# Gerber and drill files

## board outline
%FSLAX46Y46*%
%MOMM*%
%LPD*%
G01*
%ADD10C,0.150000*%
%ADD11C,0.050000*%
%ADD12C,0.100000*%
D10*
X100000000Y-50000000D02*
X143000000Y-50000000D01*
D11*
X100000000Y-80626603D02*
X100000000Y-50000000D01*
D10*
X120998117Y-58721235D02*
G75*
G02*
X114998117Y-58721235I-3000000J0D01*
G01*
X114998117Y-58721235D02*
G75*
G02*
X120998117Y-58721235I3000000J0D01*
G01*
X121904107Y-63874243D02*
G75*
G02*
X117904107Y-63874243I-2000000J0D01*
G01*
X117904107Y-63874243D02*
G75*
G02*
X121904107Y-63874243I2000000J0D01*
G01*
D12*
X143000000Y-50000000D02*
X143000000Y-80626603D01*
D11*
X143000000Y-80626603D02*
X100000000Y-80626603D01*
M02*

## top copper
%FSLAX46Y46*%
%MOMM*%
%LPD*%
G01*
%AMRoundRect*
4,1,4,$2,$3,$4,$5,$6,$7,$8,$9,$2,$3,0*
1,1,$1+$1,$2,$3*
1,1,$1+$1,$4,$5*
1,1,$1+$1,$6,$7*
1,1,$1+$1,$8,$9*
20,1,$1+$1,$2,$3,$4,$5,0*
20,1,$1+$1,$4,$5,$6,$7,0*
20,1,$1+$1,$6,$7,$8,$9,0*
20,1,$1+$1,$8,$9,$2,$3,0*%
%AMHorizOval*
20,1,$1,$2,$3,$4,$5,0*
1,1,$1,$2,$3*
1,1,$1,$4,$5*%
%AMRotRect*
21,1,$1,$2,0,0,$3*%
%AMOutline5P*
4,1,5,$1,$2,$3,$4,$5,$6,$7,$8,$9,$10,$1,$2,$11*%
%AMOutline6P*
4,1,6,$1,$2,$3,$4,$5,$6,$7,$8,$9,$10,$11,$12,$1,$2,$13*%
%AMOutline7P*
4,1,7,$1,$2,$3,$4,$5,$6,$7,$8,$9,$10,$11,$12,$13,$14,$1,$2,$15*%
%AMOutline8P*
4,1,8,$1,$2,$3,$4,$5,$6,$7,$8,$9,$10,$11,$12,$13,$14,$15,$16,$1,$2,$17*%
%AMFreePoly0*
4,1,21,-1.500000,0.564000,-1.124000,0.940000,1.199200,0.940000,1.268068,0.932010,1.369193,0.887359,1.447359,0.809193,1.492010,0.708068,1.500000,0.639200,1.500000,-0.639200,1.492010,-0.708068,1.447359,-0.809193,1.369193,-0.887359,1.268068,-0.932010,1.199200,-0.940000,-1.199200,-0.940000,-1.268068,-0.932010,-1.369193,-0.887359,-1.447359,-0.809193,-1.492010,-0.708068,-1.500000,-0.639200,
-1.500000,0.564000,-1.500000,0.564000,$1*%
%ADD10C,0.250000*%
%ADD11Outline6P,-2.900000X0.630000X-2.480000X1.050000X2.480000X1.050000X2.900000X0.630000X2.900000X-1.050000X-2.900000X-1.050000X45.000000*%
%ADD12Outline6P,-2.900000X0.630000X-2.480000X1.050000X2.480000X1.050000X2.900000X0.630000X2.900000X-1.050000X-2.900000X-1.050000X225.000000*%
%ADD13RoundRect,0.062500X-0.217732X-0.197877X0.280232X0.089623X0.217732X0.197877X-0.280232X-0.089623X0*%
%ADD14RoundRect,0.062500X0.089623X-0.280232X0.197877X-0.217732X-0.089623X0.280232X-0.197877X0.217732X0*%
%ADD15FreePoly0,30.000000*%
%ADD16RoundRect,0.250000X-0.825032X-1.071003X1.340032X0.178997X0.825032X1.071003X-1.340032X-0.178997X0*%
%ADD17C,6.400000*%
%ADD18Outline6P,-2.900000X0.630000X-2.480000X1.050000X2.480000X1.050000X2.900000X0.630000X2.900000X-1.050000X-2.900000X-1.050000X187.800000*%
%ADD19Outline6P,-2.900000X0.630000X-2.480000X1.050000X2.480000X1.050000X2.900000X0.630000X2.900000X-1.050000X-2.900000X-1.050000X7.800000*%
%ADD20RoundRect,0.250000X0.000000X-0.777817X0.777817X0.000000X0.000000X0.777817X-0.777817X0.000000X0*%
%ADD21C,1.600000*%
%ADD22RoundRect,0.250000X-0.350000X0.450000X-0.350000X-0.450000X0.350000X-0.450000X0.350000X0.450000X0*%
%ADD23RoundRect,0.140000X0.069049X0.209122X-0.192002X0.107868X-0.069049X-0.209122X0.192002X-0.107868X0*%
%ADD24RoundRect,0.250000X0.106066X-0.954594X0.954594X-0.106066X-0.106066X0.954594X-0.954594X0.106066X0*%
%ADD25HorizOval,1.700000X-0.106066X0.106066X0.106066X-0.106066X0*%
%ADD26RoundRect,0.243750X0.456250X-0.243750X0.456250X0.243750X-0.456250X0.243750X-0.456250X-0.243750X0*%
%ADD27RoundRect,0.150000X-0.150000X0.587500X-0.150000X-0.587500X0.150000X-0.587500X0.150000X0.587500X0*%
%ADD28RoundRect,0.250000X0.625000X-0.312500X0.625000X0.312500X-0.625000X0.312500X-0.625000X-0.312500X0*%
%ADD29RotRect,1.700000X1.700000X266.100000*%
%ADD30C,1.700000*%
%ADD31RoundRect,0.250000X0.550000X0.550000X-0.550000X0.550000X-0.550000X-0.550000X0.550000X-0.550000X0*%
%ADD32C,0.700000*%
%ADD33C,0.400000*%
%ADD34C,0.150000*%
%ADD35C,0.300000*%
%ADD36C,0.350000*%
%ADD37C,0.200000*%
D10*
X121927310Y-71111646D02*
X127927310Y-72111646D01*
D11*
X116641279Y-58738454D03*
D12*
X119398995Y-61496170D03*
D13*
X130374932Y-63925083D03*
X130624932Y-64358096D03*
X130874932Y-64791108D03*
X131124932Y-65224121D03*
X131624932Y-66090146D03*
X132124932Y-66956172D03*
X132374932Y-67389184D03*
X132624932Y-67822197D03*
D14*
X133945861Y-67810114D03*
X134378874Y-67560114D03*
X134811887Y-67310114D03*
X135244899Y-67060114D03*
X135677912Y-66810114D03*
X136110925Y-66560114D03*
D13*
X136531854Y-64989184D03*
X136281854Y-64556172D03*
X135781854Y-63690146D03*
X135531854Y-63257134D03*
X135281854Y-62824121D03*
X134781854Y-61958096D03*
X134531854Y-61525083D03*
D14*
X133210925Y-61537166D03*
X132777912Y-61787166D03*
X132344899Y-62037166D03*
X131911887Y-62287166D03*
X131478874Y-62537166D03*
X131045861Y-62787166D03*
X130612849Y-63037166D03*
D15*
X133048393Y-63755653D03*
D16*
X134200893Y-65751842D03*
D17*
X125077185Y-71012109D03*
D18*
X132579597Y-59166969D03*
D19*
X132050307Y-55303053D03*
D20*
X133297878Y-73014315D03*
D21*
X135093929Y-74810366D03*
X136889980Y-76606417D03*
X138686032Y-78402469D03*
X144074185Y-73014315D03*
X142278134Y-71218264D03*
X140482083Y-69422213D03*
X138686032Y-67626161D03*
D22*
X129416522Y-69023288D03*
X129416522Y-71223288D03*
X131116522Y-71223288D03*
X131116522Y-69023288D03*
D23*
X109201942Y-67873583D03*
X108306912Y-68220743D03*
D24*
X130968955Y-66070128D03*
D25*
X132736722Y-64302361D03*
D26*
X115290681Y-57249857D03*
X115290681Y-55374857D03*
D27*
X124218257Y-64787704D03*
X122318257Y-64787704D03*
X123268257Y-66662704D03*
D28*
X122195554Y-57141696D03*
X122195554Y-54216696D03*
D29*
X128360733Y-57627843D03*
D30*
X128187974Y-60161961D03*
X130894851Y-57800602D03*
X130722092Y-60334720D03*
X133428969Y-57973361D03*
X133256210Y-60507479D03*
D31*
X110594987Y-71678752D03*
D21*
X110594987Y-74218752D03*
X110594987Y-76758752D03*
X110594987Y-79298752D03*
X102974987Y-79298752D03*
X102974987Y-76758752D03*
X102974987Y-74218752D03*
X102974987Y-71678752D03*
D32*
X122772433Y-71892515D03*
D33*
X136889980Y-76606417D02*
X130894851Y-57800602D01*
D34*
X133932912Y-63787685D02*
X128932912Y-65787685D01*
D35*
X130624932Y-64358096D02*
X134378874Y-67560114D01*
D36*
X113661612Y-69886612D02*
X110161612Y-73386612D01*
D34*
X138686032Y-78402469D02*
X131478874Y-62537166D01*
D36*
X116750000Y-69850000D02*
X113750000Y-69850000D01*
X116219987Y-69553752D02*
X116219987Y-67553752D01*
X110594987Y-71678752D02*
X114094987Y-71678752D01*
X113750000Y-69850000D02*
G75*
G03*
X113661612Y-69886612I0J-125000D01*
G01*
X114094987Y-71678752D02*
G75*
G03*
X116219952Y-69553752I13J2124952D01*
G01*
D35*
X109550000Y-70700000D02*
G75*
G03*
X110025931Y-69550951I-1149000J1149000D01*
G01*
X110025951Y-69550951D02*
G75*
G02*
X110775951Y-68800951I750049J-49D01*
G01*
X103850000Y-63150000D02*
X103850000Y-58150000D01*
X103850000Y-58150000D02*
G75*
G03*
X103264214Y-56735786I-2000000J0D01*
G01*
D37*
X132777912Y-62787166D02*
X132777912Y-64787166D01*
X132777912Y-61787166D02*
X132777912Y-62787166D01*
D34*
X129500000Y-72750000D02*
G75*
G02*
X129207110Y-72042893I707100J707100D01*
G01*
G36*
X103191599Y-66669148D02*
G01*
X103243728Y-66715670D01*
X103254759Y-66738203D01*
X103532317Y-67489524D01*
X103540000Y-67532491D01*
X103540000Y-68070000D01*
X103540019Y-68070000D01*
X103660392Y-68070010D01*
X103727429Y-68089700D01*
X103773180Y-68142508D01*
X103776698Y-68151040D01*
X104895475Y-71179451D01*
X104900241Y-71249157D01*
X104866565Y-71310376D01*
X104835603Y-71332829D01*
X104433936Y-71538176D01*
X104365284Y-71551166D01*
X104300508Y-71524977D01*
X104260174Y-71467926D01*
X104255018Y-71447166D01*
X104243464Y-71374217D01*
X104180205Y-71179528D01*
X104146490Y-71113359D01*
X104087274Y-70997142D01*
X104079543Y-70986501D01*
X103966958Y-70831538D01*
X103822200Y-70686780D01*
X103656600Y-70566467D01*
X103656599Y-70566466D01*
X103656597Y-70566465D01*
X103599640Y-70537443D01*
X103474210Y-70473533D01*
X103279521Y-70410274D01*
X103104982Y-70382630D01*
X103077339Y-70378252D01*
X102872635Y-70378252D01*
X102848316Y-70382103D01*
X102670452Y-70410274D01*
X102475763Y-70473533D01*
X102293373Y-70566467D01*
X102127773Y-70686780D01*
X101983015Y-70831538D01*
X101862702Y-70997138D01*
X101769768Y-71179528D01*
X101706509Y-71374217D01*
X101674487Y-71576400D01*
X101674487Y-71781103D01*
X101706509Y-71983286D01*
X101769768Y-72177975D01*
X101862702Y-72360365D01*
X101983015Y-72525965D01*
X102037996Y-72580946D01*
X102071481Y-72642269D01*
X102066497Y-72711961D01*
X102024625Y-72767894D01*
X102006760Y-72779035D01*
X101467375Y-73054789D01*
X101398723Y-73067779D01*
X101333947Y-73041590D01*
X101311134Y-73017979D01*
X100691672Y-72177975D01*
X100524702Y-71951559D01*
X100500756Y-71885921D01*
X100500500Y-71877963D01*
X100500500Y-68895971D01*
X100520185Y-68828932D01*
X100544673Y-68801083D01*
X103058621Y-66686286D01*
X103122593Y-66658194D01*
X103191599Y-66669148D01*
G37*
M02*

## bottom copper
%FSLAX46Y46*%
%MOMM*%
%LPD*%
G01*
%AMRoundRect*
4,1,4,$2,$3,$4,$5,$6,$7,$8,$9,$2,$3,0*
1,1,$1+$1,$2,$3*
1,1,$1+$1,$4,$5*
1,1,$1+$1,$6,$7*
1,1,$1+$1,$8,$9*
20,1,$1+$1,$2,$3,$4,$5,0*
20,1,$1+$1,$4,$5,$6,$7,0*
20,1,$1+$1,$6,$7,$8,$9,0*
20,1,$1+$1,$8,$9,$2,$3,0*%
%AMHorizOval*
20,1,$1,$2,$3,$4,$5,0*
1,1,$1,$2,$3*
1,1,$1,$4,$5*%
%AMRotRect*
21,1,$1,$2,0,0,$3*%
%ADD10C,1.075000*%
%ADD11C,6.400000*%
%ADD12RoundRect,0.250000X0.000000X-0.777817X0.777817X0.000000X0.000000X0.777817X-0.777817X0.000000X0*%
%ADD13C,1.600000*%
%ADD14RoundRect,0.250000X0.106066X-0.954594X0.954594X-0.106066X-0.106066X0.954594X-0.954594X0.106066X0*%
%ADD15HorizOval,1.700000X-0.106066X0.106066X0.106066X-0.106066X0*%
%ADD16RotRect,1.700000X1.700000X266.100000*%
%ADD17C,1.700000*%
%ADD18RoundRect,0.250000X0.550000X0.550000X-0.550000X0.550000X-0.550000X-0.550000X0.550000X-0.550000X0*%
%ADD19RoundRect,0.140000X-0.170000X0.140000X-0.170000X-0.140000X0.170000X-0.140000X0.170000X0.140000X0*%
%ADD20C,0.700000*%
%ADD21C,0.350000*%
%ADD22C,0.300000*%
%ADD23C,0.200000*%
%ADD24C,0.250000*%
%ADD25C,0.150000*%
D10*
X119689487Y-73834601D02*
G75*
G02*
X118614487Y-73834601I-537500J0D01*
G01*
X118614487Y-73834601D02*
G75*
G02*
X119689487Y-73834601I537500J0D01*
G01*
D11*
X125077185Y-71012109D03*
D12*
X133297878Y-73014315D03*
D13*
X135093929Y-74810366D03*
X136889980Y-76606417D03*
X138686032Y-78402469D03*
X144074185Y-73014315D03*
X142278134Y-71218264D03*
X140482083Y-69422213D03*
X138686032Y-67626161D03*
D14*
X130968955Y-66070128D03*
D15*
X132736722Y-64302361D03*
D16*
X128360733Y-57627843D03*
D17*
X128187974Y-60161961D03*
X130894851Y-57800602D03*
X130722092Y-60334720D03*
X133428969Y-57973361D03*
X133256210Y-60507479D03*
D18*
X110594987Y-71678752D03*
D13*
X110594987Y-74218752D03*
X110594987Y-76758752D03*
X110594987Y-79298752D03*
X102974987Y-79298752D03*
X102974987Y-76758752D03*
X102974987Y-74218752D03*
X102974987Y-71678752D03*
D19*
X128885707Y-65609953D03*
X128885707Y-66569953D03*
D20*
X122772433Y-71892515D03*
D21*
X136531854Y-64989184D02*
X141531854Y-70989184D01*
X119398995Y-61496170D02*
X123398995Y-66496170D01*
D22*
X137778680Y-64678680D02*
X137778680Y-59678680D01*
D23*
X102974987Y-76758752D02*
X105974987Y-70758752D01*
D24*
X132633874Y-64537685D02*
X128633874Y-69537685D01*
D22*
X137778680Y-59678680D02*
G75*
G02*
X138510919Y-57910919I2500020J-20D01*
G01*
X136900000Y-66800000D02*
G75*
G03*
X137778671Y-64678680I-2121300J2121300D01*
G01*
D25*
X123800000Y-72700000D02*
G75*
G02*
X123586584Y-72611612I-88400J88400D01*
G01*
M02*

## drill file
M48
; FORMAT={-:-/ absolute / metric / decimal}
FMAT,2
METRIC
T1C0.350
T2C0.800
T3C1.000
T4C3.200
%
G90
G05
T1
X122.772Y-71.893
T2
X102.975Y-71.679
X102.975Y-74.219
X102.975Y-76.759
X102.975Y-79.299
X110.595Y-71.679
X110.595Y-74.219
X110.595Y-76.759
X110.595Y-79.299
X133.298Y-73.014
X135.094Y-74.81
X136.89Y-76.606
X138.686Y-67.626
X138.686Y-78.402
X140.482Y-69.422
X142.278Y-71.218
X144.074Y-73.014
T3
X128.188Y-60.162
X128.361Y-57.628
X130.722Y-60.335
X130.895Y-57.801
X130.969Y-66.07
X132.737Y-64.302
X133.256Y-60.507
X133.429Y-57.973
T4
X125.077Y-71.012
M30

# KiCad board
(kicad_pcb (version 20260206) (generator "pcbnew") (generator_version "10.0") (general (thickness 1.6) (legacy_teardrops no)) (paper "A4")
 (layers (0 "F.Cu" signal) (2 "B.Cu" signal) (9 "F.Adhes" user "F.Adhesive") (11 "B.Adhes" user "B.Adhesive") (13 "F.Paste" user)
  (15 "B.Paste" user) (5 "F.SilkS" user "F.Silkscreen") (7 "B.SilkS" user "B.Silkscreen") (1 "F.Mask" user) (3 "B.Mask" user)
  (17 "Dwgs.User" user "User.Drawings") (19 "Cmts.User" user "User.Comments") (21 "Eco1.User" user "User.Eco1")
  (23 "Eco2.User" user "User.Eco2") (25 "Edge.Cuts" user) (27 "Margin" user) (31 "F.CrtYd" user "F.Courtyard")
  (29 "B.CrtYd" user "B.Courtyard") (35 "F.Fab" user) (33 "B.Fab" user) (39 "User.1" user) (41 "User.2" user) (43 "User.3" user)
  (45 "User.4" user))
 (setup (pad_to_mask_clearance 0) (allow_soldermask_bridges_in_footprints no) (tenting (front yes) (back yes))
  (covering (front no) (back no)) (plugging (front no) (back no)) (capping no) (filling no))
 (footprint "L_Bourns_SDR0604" (layer "F.Cu") (at 118.020137 60.117312 45)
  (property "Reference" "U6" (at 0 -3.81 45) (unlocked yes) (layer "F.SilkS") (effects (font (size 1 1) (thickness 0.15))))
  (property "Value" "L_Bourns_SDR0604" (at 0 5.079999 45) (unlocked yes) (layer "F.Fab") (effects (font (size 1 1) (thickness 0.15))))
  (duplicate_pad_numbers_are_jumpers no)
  (pad "1" smd roundrect (at 0 -1.95 45) (size 5.8 2.1) (layers "F.Cu" "F.Mask" "F.Paste") (roundrect_rratio 0) (chamfer_ratio 0.2)
   (chamfer top_left top_right) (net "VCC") (die_length 2))
  (pad "2" smd roundrect (at 0 1.95 225) (size 5.8 2.1) (layers "F.Cu" "F.Mask" "F.Paste") (roundrect_rratio 0) (chamfer_ratio 0.2)
   (chamfer top_left top_right) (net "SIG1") (die_length 2)))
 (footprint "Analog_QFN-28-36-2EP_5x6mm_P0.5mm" (layer "F.Cu") (at 133.578393 64.67364 30)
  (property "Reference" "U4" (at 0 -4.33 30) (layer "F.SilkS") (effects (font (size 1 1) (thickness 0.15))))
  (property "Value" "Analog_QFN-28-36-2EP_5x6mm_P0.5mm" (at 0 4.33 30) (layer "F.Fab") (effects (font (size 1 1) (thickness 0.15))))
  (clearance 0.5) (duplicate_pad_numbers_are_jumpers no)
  (pad "" smd roundrect (at -0.75 -1.53 30) (size 1.21 0.76) (layers "F.Paste") (roundrect_rratio 0.25) (chamfer_ratio 0.4)
   (chamfer top_left) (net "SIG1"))
  (pad "" smd roundrect (at -0.75 -0.59 30) (size 1.21 0.76) (layers "F.Paste") (roundrect_rratio 0.25) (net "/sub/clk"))
  (pad "" smd roundrect (at -0.7475 0.875 30) (size 1.205 0.55) (layers "F.Paste") (roundrect_rratio 0.25) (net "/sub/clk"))
  (pad "" smd roundrect (at -0.7475 1.625 30) (size 1.205 0.55) (layers "F.Paste") (roundrect_rratio 0.25) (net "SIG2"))
  (pad "" smd roundrect (at 0.7475 0.875 30) (size 1.205 0.55) (layers "F.Paste") (roundrect_rratio 0.25) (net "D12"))
  (pad "" smd roundrect (at 0.7475 1.625 30) (size 1.205 0.55) (layers "F.Paste") (roundrect_rratio 0.25))
  (pad "" smd roundrect (at 0.75 -1.53 30) (size 1.21 0.76) (layers "F.Paste") (roundrect_rratio 0.25) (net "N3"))
  (pad "" smd roundrect (at 0.75 -0.59 30) (size 1.21 0.76) (layers "F.Paste") (roundrect_rratio 0.25))
  (pad "1" smd roundrect (at -2.4 -2.25 30) (size 0.7 0.25) (layers "F.Cu" "F.Mask" "F.Paste") (roundrect_rratio 0.25) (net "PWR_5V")
   (clearance 0.35))
  (pad "2" smd roundrect (at -2.4 -1.75 30) (size 0.7 0.25) (layers "F.Cu" "F.Mask" "F.Paste") (roundrect_rratio 0.25))
  (pad "3" smd roundrect (at -2.4 -1.25 30) (size 0.7 0.25) (layers "F.Cu" "F.Mask" "F.Paste") (roundrect_rratio 0.25) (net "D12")
   (clearance 0.1))
  (pad "4" smd roundrect (at -2.4 -0.75 30) (size 0.7 0.25) (layers "F.Cu" "F.Mask" "F.Paste") (roundrect_rratio 0.25) (clearance 0.35))
  (pad "6" smd roundrect (at -2.4 0.25 30) (size 0.7 0.25) (layers "F.Cu" "F.Mask" "F.Paste") (roundrect_rratio 0.25) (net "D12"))
  (pad "8" smd roundrect (at -2.4 1.25 30) (size 0.7 0.25) (layers "F.Cu" "F.Mask" "F.Paste") (roundrect_rratio 0.25) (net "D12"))
  (pad "9" smd roundrect (at -2.4 1.75 30) (size 0.7 0.25) (layers "F.Cu" "F.Mask" "F.Paste") (roundrect_rratio 0.25) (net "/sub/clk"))
  (pad "10" smd roundrect (at -2.4 2.25 30) (size 0.7 0.25) (layers "F.Cu" "F.Mask" "F.Paste") (roundrect_rratio 0.25) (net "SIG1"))
  (pad "12" smd roundrect (at -1.25 2.9 30) (size 0.25 0.7) (layers "F.Cu" "F.Mask" "F.Paste") (roundrect_rratio 0.25) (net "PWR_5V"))
  (pad "13" smd roundrect (at -0.75 2.9 30) (size 0.25 0.7) (layers "F.Cu" "F.Mask" "F.Paste") (roundrect_rratio 0.25) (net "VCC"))
  (pad "14" smd roundrect (at -0.25 2.9 30) (size 0.25 0.7) (layers "F.Cu" "F.Mask" "F.Paste") (roundrect_rratio 0.25) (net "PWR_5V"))
  (pad "15" smd roundrect (at 0.25 2.9 30) (size 0.25 0.7) (layers "F.Cu" "F.Mask" "F.Paste") (roundrect_rratio 0.25) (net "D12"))
  (pad "16" smd roundrect (at 0.75 2.9 30) (size 0.25 0.7) (layers "F.Cu" "F.Mask" "F.Paste") (roundrect_rratio 0.25) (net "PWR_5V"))
  (pad "17" smd roundrect (at 1.25 2.9 30) (size 0.25 0.7) (layers "F.Cu" "F.Mask" "F.Paste") (roundrect_rratio 0.25))
  (pad "20" smd roundrect (at 2.4 1.75 30) (size 0.7 0.25) (layers "F.Cu" "F.Mask" "F.Paste") (roundrect_rratio 0.25))
  (pad "21" smd roundrect (at 2.4 1.25 30) (size 0.7 0.25) (layers "F.Cu" "F.Mask" "F.Paste") (roundrect_rratio 0.25) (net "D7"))
  (pad "23" smd roundrect (at 2.4 0.25 30) (size 0.7 0.25) (layers "F.Cu" "F.Mask" "F.Paste") (roundrect_rratio 0.25) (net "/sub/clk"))
  (pad "24" smd roundrect (at 2.4 -0.25 30) (size 0.7 0.25) (layers "F.Cu" "F.Mask" "F.Paste") (roundrect_rratio 0.25) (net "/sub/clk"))
  (pad "25" smd roundrect (at 2.4 -0.75 30) (size 0.7 0.25) (layers "F.Cu" "F.Mask" "F.Paste") (roundrect_rratio 0.25) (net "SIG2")
   (clearance 0.1))
  (pad "27" smd roundrect (at 2.4 -1.75 30) (size 0.7 0.25) (layers "F.Cu" "F.Mask" "F.Paste") (roundrect_rratio 0.25))
  (pad "28" smd roundrect (at 2.4 -2.25 30) (size 0.7 0.25) (layers "F.Cu" "F.Mask" "F.Paste") (roundrect_rratio 0.25) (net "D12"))
  (pad "30" smd roundrect (at 1.25 -2.9 30) (size 0.25 0.7) (layers "F.Cu" "F.Mask" "F.Paste") (roundrect_rratio 0.25) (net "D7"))
  (pad "31" smd roundrect (at 0.75 -2.9 30) (size 0.25 0.7) (layers "F.Cu" "F.Mask" "F.Paste") (roundrect_rratio 0.25))
  (pad "32" smd roundrect (at 0.25 -2.9 30) (size 0.25 0.7) (layers "F.Cu" "F.Mask" "F.Paste") (roundrect_rratio 0.25) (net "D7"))
  (pad "33" smd roundrect (at -0.25 -2.9 30) (size 0.25 0.7) (layers "F.Cu" "F.Mask" "F.Paste") (roundrect_rratio 0.25) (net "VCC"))
  (pad "34" smd roundrect (at -0.75 -2.9 30) (size 0.25 0.7) (layers "F.Cu" "F.Mask" "F.Paste") (roundrect_rratio 0.25) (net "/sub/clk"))
  (pad "35" smd roundrect (at -1.25 -2.9 30) (size 0.25 0.7) (layers "F.Cu" "F.Mask" "F.Paste") (roundrect_rratio 0.25) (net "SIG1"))
  (pad "36" smd roundrect (at -1.749999 -2.9 30) (size 0.25 0.7) (layers "F.Cu" "F.Mask" "F.Paste") (roundrect_rratio 0.25) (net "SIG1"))
  (pad "37" smd roundrect (at 0 -1.06 30) (size 3 1.88) (layers "F.Cu" "F.Mask") (roundrect_rratio 0.16) (chamfer_ratio 0.2)
   (chamfer top_left) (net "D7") (zone_connect 2))
  (pad "38" smd roundrect (at 0 1.245 30) (size 3 1.53) (layers "F.Cu" "F.Mask") (roundrect_rratio 0.1633986928) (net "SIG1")
   (zone_connect 2)))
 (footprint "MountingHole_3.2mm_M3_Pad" (layer "F.Cu") (at 125.077185 71.012109)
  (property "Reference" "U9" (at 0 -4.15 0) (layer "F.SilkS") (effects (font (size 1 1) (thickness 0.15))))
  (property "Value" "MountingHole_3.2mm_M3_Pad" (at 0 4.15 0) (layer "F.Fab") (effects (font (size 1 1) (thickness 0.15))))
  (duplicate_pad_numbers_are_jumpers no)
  (pad "1" thru_hole circle (at 0 0) (size 6.4 6.4) (drill 3.2) (layers "*.Cu" "*.Mask") (remove_unused_layers no) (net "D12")
   (zone_connect 2))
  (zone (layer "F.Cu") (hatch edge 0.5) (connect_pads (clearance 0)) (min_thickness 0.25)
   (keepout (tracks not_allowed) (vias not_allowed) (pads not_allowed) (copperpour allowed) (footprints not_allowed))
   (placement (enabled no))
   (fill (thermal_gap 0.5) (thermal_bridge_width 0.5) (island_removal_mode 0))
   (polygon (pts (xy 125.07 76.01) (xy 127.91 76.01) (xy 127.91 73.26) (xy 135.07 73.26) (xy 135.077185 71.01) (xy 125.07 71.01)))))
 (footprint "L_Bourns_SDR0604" (layer "F.Cu") (at 132.314952 57.235011 -172.2)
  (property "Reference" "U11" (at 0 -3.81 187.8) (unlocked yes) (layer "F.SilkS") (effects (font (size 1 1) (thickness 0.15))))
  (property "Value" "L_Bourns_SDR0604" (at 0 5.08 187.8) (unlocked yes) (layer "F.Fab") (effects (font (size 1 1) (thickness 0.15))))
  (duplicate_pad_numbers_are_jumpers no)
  (pad "1" smd roundrect (at 0 -1.95 187.8) (size 5.8 2.1) (layers "F.Cu" "F.Mask" "F.Paste") (roundrect_rratio 0) (chamfer_ratio 0.2)
   (chamfer top_left top_right) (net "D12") (die_length 2))
  (pad "2" smd roundrect (at 0 1.95 7.8) (size 5.8 2.1) (layers "F.Cu" "F.Mask" "F.Paste") (roundrect_rratio 0) (chamfer_ratio 0.2)
   (chamfer top_left top_right) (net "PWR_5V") (die_length 2)))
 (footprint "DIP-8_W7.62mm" (layer "F.Cu") (at 133.297878 73.014315 45)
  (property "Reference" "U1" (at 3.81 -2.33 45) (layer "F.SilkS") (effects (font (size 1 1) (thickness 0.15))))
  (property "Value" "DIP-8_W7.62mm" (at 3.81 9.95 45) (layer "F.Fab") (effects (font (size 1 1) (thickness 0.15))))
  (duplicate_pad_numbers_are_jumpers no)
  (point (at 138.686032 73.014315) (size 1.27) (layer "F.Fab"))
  (pad "1" thru_hole roundrect (at 0 0 45) (size 1.6 1.6) (drill 0.8) (layers "*.Cu" "*.Mask") (remove_unused_layers no)
   (roundrect_rratio 0.15625) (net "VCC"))
  (pad "2" thru_hole circle (at 0 2.54 45) (size 1.6 1.6) (drill 0.8) (layers "*.Cu" "*.Mask") (remove_unused_layers no) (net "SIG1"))
  (pad "3" thru_hole circle (at 0 5.079999 45) (size 1.6 1.6) (drill 0.8) (layers "*.Cu" "*.Mask") (remove_unused_layers no))
  (pad "4" thru_hole circle (at 0 7.62 45) (size 1.6 1.6) (drill 0.8) (layers "*.Cu" "*.Mask") (remove_unused_layers no) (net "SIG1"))
  (pad "5" thru_hole circle (at 7.62 7.62 45) (size 1.6 1.6) (drill 0.8) (layers "*.Cu" "*.Mask") (remove_unused_layers no))
  (pad "6" thru_hole circle (at 7.62 5.08 45) (size 1.6 1.6) (drill 0.8) (layers "*.Cu" "*.Mask") (remove_unused_layers no) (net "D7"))
  (pad "7" thru_hole circle (at 7.62 2.54 45) (size 1.6 1.6) (drill 0.8) (layers "*.Cu" "*.Mask") (remove_unused_layers no) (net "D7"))
  (pad "8" thru_hole circle (at 7.62 0 45) (size 1.6 1.6) (drill 0.8) (layers "*.Cu" "*.Mask") (remove_unused_layers no) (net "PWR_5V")))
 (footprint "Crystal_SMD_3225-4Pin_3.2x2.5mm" (layer "F.Cu") (at 130.266522 70.123288 -90)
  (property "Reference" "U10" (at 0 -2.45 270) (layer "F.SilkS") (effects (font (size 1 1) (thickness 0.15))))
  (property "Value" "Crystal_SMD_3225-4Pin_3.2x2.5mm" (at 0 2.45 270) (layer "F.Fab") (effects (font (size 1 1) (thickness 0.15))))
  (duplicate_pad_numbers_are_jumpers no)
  (pad "1" smd roundrect (at -1.1 0.85 270) (size 1.4 1.2) (layers "F.Cu" "F.Mask" "F.Paste") (roundrect_rratio 0.208333) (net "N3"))
  (pad "2" smd roundrect (at 1.1 0.85 270) (size 1.4 1.2) (layers "F.Cu" "F.Mask" "F.Paste") (roundrect_rratio 0.208333))
  (pad "3" smd roundrect (at 1.1 -0.85 270) (size 1.4 1.2) (layers "F.Cu" "F.Mask" "F.Paste") (roundrect_rratio 0.208333) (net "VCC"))
  (pad "4" smd roundrect (at -1.1 -0.85 270) (size 1.4 1.2) (layers "F.Cu" "F.Mask" "F.Paste") (roundrect_rratio 0.208333) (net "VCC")))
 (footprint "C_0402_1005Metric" (layer "F.Cu") (at 108.754427 68.047163 -158.8)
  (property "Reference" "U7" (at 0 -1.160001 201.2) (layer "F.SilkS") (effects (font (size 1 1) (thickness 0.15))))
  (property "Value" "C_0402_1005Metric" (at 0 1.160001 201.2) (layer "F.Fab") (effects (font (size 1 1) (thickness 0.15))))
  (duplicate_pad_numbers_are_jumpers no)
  (pad "1" smd roundrect (at -0.48 0 201.2) (size 0.56 0.62) (layers "F.Cu" "F.Mask" "F.Paste") (roundrect_rratio 0.25) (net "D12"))
  (pad "2" smd roundrect (at 0.48 0 201.2) (size 0.56 0.62) (layers "F.Cu" "F.Mask" "F.Paste") (roundrect_rratio 0.25) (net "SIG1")))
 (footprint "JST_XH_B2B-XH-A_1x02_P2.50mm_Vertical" (layer "F.Cu") (at 130.968955 66.070128 45)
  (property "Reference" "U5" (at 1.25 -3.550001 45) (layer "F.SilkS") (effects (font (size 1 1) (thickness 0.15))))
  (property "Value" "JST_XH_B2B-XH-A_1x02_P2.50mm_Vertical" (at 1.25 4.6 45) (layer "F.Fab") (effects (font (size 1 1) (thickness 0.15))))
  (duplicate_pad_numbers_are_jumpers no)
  (pad "1" thru_hole roundrect (at 0 0 45) (size 1.7 2) (drill 1) (layers "*.Cu" "*.Mask") (remove_unused_layers no)
   (roundrect_rratio 0.147059))
  (pad "2" thru_hole oval (at 2.5 0 45) (size 1.7 2) (drill 1) (layers "*.Cu" "*.Mask") (remove_unused_layers no) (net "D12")))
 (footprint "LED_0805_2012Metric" (layer "F.Cu") (at 115.290681 56.312357 90)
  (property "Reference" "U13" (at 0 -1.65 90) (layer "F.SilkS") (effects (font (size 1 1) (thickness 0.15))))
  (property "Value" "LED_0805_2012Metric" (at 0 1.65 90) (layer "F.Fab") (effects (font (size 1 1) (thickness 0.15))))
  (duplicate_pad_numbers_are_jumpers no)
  (pad "1" smd roundrect (at -0.9375 0 90) (size 0.975 1.4) (layers "F.Cu" "F.Mask" "F.Paste") (roundrect_rratio 0.25))
  (pad "2" smd roundrect (at 0.9375 0 90) (size 0.975 1.4) (layers "F.Cu" "F.Mask" "F.Paste") (roundrect_rratio 0.25) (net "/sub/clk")))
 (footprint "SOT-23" (layer "F.Cu") (at 123.268257 65.725204 -90)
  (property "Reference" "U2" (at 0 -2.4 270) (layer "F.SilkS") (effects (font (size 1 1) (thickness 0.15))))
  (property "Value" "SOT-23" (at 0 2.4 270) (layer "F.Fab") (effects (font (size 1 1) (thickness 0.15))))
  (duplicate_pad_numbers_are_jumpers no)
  (pad "1" smd roundrect (at -0.9375 -0.95 270) (size 1.475 0.6) (layers "F.Cu" "F.Mask" "F.Paste") (roundrect_rratio 0.25) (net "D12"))
  (pad "2" smd roundrect (at -0.9375 0.95 270) (size 1.475 0.6) (layers "F.Cu" "F.Mask" "F.Paste") (roundrect_rratio 0.25) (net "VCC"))
  (pad "3" smd roundrect (at 0.9375 0 270) (size 1.475 0.6) (layers "F.Cu" "F.Mask" "F.Paste") (roundrect_rratio 0.25)))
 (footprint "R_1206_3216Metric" (layer "F.Cu") (at 122.195554 55.679196 90)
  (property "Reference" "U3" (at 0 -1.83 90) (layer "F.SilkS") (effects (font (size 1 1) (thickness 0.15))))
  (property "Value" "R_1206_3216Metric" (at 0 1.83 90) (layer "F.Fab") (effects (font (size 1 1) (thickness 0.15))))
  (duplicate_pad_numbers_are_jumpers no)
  (pad "1" smd roundrect (at -1.4625 0 90) (size 1.125 1.75) (layers "F.Cu" "F.Mask" "F.Paste") (roundrect_rratio 0.222222) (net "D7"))
  (pad "2" smd roundrect (at 1.4625 0 90) (size 1.125 1.75) (layers "F.Cu" "F.Mask" "F.Paste") (roundrect_rratio 0.222222)))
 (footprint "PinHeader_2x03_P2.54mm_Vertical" (layer "B.Cu") (at 128.360733 57.627843 -93.9)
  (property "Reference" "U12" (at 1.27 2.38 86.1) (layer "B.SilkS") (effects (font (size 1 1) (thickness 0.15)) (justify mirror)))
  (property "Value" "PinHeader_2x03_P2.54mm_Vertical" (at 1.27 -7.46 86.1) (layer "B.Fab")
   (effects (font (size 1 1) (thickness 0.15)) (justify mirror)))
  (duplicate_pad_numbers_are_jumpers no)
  (pad "1" thru_hole rect (at 0 0 266.1) (size 1.7 1.7) (drill 1) (layers "*.Cu" "*.Mask") (remove_unused_layers no) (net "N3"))
  (pad "2" thru_hole circle (at 2.54 0 266.1) (size 1.7 1.7) (drill 1) (layers "*.Cu" "*.Mask") (remove_unused_layers no) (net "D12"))
  (pad "3" thru_hole circle (at 0 -2.54 266.1) (size 1.7 1.7) (drill 1) (layers "*.Cu" "*.Mask") (remove_unused_layers no) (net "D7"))
  (pad "4" thru_hole circle (at 2.54 -2.54 266.1) (size 1.7 1.7) (drill 1) (layers "*.Cu" "*.Mask") (remove_unused_layers no) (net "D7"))
  (pad "5" thru_hole circle (at 0 -5.08 266.1) (size 1.7 1.7) (drill 1) (layers "*.Cu" "*.Mask") (remove_unused_layers no) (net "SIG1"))
  (pad "6" thru_hole circle (at 2.54 -5.08 266.1) (size 1.7 1.7) (drill 1) (layers "*.Cu" "*.Mask") (remove_unused_layers no) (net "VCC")))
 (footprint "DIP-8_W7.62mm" (layer "B.Cu") (at 110.594987 71.678752 180)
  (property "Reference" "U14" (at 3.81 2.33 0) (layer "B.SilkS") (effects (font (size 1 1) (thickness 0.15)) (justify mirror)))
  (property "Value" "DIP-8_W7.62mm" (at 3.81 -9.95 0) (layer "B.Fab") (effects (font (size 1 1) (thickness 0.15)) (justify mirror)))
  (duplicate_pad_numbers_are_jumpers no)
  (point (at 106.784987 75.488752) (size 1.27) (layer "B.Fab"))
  (pad "1" thru_hole roundrect (at 0 0 180) (size 1.6 1.6) (drill 0.8) (layers "*.Cu" "*.Mask") (remove_unused_layers no)
   (roundrect_rratio 0.15625) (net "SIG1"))
  (pad "2" thru_hole circle (at 0 -2.54 180) (size 1.6 1.6) (drill 0.8) (layers "*.Cu" "*.Mask") (remove_unused_layers no) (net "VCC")
   (clearance 0.1))
  (pad "3" thru_hole circle (at 0 -5.08 180) (size 1.6 1.6) (drill 0.8) (layers "*.Cu" "*.Mask") (remove_unused_layers no))
  (pad "4" thru_hole circle (at 0 -7.62 180) (size 1.6 1.6) (drill 0.8) (layers "*.Cu" "*.Mask") (remove_unused_layers no))
  (pad "5" thru_hole circle (at 7.62 -7.62 180) (size 1.6 1.6) (drill 0.8) (layers "*.Cu" "*.Mask") (remove_unused_layers no) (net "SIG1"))
  (pad "6" thru_hole circle (at 7.62 -5.08 180) (size 1.6 1.6) (drill 0.8) (layers "*.Cu" "*.Mask") (remove_unused_layers no)
   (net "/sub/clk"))
  (pad "7" thru_hole circle (at 7.62 -2.54 180) (size 1.6 1.6) (drill 0.8) (layers "*.Cu" "*.Mask") (remove_unused_layers no) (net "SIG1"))
  (pad "8" thru_hole circle (at 7.62 0 180) (size 1.6 1.6) (drill 0.8) (layers "*.Cu" "*.Mask") (remove_unused_layers no) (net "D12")))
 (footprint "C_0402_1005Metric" (layer "B.Cu") (at 128.885707 66.089953 -90)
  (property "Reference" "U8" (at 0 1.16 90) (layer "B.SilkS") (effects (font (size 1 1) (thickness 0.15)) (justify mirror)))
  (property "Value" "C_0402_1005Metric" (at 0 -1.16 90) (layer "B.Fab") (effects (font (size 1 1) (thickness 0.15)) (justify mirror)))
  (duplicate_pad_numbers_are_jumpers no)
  (pad "1" smd roundrect (at -0.48 0 270) (size 0.56 0.62) (layers "B.Cu" "B.Mask" "B.Paste") (roundrect_rratio 0.25) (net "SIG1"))
  (pad "2" smd roundrect (at 0.48 0 270) (size 0.56 0.62) (layers "B.Cu" "B.Mask" "B.Paste") (roundrect_rratio 0.25) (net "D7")))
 (gr_line (start 121.92731 71.111646) (end 127.92731 72.111646) (stroke (width 0.25) (type default)) (layer "F.Cu") (net "D12"))
 (gr_circle (center 119.151987 73.834601) (end 120.151987 73.834601) (stroke (width 0.15) (type default)) (fill yes) (layer "B.Cu")
  (net "SIG1"))
 (gr_line (start 100 50) (end 143 50) (stroke (width 0.15) (type default)) (layer "Edge.Cuts"))
 (gr_line (start 100 80.626603) (end 100 50) (stroke (width 0.05) (type default)) (layer "Edge.Cuts"))
 (gr_circle (center 117.998117 58.721235) (end 120.998117 58.721235) (stroke (width 0.15) (type default)) (fill no) (layer "Edge.Cuts"))
 (gr_circle (center 119.904107 63.874243) (end 121.904107 63.874243) (stroke (width 0.15) (type default)) (fill no) (layer "Edge.Cuts"))
 (gr_line (start 143 50) (end 143 80.626603) (stroke (width 0.1) (type default)) (layer "Edge.Cuts"))
 (gr_line (start 143 80.626603) (end 100 80.626603) (stroke (width 0.05) (type default)) (layer "Edge.Cuts"))
 (segment (start 136.88998 76.606417) (end 130.894851 57.800602) (width 0.4) (layer "F.Cu") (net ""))
 (segment (start 133.932912 63.787685) (end 128.932912 65.787685) (width 0.15) (layer "F.Cu") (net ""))
 (segment (start 130.624932 64.358096) (end 134.378874 67.560114) (width 0.3) (layer "F.Cu") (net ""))
 (segment (start 136.531854 64.989184) (end 141.531854 70.989184) (width 0.35) (layer "B.Cu") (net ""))
 (via (at 122.772433 71.892515) (size 0.7) (drill 0.35) (layers "F.Cu" "B.Cu") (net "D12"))
 (segment (start 113.661612 69.886612) (end 110.161612 73.386612) (width 0.35) (layer "F.Cu") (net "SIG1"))
 (segment (start 138.686032 78.402469) (end 131.478874 62.537166) (width 0.15) (layer "F.Cu") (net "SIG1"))
 (segment (start 116.75 69.85) (end 113.75 69.85) (width 0.35) (layer "F.Cu") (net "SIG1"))
 (segment (start 116.219987 69.553752) (end 116.219987 67.553752) (width 0.35) (layer "F.Cu") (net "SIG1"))
 (segment (start 110.594987 71.678752) (end 114.094987 71.678752) (width 0.35) (layer "F.Cu") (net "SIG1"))
 (arc (start 113.75 69.85) (mid 113.702165 69.859515) (end 113.661612 69.886612) (width 0.35) (layer "F.Cu") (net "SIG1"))
 (arc (start 114.094987 71.678752) (mid 115.597589 71.056354) (end 116.219987 69.553752) (width 0.35) (layer "F.Cu") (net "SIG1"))
 (arc (start 109.55 70.7) (mid 109.902256 70.172812) (end 110.025951 69.550951) (width 0.3) (layer "F.Cu") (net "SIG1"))
 (arc (start 110.025951 69.550951) (mid 110.245621 69.020621) (end 110.775951 68.800951) (width 0.3) (layer "F.Cu") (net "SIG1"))
 (segment (start 119.398995 61.49617) (end 123.398995 66.49617) (width 0.35) (layer "B.Cu") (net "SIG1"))
 (segment (start 103.85 63.15) (end 103.85 58.15) (width 0.3) (layer "F.Cu") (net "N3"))
 (arc (start 103.85 58.15) (mid 103.697759 57.384633) (end 103.264214 56.735786) (width 0.3) (layer "F.Cu") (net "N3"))
 (segment (start 137.77868 64.67868) (end 137.77868 59.67868) (width 0.3) (layer "B.Cu") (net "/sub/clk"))
 (segment (start 102.974987 76.758752) (end 105.974987 70.758752) (width 0.2) (layer "B.Cu") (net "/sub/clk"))
 (segment (start 132.633874 64.537685) (end 128.633874 69.537685) (width 0.25) (layer "B.Cu") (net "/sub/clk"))
 (arc (start 137.77868 59.67868) (mid 137.968981 58.721971) (end 138.510913 57.910913) (width 0.3) (layer "B.Cu") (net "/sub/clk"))
 (arc (start 136.9 66.8) (mid 137.550318 65.82673) (end 137.77868 64.67868) (width 0.3) (layer "B.Cu") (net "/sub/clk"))
 (arc (start 123.8 72.7) (mid 123.663776 72.727097) (end 123.586612 72.611612) (width 0.15) (layer "B.Cu") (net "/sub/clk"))
 (segment (start 132.777912 62.787166) (end 132.777912 64.787166) (width 0.2) (layer "F.Cu") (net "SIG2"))
 (segment (start 132.777912 61.787166) (end 132.777912 62.787166) (width 0.2) (layer "F.Cu") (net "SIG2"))
 (arc (start 129.5 72.75) (mid 129.283227 72.425577) (end 129.207107 72.042893) (width 0.15) (layer "F.Cu") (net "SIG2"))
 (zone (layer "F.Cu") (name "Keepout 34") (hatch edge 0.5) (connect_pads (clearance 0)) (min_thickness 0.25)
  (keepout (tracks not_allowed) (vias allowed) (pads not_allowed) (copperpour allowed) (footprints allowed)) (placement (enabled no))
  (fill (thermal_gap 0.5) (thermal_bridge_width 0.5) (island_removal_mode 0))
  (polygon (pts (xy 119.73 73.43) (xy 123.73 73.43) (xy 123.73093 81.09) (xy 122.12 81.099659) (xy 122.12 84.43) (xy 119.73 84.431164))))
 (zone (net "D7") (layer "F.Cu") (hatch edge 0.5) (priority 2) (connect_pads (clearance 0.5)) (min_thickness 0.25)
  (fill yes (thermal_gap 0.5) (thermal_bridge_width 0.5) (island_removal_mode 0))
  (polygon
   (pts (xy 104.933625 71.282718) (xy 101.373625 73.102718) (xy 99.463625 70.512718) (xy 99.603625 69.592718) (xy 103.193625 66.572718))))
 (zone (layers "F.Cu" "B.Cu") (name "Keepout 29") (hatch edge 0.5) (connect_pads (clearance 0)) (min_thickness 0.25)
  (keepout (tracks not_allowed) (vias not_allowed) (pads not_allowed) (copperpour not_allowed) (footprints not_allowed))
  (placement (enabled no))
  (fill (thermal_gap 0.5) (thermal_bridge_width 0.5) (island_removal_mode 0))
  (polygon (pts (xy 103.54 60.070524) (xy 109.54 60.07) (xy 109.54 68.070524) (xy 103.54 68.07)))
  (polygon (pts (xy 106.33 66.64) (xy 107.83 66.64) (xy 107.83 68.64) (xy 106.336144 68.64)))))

